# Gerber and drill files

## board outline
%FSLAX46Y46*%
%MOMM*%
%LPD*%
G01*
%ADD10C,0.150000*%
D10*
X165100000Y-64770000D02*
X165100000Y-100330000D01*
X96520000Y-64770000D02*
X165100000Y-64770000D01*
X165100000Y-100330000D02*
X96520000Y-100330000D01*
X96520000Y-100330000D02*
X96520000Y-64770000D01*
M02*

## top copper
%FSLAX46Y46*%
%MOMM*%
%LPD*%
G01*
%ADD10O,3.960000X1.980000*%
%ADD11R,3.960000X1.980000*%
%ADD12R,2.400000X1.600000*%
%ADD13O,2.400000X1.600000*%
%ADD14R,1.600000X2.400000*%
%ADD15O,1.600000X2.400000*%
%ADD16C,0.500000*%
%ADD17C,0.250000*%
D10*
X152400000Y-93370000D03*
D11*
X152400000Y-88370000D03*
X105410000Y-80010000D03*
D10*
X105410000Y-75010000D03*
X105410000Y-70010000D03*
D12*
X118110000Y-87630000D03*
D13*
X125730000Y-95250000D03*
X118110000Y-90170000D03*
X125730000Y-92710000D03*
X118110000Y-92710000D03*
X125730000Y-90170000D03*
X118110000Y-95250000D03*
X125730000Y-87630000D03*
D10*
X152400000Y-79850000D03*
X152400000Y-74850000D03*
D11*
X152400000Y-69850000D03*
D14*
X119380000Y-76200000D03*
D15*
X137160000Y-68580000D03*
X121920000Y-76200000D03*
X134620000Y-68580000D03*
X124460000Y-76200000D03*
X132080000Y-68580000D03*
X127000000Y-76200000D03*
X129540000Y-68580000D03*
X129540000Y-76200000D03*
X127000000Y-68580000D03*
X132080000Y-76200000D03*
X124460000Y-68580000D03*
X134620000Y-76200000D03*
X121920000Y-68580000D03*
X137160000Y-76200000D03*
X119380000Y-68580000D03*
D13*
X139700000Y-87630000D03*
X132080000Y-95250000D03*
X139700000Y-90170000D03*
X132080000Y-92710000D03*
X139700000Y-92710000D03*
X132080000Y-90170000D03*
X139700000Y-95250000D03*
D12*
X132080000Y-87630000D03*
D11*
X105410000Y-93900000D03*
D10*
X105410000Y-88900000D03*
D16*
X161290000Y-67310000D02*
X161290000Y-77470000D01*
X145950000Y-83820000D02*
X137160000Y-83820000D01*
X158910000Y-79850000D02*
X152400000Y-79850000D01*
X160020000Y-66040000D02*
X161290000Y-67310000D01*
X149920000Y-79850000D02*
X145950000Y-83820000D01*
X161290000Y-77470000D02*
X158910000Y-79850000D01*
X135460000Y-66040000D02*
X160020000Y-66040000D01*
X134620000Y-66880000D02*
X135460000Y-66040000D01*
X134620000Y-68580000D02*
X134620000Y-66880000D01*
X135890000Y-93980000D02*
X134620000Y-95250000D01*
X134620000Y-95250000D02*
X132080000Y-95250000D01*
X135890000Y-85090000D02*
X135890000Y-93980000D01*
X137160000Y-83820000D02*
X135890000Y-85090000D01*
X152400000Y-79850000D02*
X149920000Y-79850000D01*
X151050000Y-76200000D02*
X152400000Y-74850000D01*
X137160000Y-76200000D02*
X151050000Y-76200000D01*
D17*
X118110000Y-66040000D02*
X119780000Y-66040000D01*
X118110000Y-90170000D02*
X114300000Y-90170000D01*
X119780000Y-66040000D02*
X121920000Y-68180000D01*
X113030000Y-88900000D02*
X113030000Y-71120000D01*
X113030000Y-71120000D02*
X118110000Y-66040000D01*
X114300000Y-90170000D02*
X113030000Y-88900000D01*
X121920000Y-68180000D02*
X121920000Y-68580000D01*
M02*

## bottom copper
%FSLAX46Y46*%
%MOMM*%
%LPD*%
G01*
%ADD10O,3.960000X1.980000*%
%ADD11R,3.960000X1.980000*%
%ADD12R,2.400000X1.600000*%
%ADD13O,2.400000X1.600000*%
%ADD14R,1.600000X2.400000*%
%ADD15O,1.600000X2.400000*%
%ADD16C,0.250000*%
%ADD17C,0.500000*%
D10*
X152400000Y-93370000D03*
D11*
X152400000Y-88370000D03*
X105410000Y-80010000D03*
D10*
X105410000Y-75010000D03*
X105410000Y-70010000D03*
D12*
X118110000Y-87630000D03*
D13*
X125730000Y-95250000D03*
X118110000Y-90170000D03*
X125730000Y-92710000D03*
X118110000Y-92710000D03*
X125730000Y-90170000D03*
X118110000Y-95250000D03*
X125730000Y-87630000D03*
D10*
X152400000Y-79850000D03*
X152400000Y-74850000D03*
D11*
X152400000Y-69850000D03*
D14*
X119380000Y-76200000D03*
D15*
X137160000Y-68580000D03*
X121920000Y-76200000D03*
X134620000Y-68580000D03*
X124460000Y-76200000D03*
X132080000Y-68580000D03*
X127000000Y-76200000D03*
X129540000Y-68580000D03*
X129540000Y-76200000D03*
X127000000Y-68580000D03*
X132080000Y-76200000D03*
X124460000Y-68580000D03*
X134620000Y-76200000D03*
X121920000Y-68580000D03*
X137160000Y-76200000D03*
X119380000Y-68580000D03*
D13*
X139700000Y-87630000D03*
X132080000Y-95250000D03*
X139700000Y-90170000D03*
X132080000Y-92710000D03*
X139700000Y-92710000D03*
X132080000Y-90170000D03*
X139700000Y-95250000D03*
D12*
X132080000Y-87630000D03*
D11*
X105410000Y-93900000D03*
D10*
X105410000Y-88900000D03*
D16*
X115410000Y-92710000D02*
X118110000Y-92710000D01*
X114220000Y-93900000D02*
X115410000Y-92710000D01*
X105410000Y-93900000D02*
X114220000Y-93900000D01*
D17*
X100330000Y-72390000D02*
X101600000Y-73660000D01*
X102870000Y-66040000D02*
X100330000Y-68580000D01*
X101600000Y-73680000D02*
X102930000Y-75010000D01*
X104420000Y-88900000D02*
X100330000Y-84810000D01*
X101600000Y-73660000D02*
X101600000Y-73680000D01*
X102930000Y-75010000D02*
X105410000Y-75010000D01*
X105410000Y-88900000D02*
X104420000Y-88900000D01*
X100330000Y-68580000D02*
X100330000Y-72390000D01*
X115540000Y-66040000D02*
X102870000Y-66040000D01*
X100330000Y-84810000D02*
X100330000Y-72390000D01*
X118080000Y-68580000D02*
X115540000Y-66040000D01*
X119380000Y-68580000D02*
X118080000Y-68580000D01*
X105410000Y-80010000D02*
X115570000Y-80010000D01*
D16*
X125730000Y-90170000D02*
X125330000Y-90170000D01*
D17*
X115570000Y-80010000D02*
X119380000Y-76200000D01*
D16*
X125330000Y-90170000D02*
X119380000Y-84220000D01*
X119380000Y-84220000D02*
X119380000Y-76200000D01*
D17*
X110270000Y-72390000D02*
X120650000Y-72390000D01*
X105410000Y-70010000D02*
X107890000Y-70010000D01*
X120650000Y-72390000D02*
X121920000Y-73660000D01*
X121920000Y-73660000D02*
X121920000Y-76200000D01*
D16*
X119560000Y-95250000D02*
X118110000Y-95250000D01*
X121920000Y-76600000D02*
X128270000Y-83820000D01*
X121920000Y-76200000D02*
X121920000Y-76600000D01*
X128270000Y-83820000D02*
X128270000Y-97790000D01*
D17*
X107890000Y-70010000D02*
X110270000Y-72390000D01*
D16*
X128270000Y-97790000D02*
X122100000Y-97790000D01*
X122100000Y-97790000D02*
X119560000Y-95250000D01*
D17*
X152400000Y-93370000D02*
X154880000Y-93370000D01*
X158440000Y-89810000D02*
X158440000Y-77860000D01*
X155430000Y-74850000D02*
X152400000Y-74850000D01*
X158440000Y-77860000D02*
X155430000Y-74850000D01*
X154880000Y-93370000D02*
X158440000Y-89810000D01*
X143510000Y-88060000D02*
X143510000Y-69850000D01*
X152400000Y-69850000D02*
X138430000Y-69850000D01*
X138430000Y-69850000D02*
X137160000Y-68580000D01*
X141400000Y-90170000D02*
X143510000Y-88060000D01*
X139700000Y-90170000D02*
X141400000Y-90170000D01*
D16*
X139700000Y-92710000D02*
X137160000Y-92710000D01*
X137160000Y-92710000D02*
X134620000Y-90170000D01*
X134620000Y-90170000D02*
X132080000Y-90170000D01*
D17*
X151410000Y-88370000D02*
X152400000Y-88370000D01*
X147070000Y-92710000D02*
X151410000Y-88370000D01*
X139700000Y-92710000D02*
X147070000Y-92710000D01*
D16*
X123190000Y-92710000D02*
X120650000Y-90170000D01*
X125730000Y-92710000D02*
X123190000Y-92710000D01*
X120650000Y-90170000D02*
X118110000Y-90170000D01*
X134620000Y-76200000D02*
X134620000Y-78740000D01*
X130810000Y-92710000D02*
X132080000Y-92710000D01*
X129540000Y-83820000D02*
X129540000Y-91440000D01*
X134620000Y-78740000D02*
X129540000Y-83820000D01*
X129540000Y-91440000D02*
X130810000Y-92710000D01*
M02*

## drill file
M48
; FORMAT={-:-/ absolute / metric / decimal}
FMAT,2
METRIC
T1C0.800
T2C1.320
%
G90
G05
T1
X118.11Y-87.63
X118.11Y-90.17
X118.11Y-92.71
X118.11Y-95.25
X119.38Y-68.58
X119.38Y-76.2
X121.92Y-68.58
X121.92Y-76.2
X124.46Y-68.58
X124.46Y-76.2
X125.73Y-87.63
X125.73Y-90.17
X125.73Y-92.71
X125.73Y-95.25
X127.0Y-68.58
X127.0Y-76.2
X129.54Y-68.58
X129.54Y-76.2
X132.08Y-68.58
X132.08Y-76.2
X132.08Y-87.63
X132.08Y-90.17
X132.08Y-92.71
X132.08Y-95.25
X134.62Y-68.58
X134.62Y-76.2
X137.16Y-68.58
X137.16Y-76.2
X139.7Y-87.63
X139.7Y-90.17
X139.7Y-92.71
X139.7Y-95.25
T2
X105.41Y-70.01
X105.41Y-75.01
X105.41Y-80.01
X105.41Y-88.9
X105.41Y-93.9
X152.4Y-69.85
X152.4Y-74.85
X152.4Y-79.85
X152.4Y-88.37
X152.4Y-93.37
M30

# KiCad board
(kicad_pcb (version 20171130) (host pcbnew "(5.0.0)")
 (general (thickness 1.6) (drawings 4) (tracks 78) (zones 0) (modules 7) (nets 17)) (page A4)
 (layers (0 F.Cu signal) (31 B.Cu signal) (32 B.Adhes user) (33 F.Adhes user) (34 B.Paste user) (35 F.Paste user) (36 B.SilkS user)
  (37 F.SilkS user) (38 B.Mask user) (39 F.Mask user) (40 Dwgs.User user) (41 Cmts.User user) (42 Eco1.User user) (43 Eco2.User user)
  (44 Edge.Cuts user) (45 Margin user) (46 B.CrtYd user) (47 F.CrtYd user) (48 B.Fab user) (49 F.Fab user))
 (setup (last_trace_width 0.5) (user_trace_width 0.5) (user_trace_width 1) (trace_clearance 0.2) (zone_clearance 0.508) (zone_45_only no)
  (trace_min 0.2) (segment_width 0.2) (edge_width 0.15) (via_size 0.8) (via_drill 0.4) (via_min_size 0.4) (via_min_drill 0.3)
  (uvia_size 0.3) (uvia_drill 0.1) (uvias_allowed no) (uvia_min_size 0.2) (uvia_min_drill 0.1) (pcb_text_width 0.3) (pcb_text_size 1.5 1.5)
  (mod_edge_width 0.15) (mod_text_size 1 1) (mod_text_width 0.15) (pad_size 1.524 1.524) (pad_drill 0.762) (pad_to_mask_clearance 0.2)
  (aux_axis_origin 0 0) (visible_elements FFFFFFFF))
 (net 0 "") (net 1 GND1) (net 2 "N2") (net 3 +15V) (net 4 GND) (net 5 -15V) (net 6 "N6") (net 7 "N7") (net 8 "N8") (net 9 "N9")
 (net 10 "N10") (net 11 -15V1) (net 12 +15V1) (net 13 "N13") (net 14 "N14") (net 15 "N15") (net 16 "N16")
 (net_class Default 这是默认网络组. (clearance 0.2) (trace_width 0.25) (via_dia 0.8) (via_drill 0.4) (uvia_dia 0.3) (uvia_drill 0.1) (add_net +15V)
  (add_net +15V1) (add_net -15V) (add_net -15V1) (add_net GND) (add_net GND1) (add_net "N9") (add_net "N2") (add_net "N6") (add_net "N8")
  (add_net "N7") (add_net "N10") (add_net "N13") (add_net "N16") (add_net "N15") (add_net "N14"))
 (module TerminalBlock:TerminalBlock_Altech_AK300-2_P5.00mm (layer F.Cu) (at 152.4 88.37 270)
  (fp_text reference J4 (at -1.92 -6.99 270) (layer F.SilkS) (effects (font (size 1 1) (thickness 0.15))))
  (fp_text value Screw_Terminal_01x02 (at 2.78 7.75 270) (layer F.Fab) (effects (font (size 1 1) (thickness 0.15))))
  (pad 2 thru_hole oval (at 5 0 270) (size 1.98 3.96) (drill 1.32) (layers *.Cu *.Mask) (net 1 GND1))
  (pad 1 thru_hole rect (at 0 0 270) (size 1.98 3.96) (drill 1.32) (layers *.Cu *.Mask) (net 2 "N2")))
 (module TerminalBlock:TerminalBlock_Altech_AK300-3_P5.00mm (layer F.Cu) (at 105.41 80.01 90)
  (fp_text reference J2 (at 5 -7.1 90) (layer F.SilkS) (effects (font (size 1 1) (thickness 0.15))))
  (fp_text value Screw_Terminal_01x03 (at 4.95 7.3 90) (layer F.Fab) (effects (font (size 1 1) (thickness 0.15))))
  (pad 1 thru_hole rect (at 0 0 90) (size 1.98 3.96) (drill 1.32) (layers *.Cu *.Mask) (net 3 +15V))
  (pad 2 thru_hole oval (at 5 0 90) (size 1.98 3.96) (drill 1.32) (layers *.Cu *.Mask) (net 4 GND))
  (pad 3 thru_hole oval (at 10 0 90) (size 1.98 3.96) (drill 1.32) (layers *.Cu *.Mask) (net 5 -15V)))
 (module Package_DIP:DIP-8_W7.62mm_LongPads (layer F.Cu) (at 118.11 87.63)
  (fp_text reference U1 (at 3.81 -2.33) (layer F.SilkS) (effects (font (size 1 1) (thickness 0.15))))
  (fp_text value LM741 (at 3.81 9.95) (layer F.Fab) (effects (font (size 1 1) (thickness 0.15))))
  (pad 1 thru_hole rect (at 0 0) (size 2.4 1.6) (drill 0.8) (layers *.Cu *.Mask) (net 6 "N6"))
  (pad 5 thru_hole oval (at 7.62 7.62) (size 2.4 1.6) (drill 0.8) (layers *.Cu *.Mask) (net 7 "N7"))
  (pad 2 thru_hole oval (at 0 2.54) (size 2.4 1.6) (drill 0.8) (layers *.Cu *.Mask) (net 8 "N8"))
  (pad 6 thru_hole oval (at 7.62 5.08) (size 2.4 1.6) (drill 0.8) (layers *.Cu *.Mask) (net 8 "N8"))
  (pad 3 thru_hole oval (at 0 5.08) (size 2.4 1.6) (drill 0.8) (layers *.Cu *.Mask) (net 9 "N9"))
  (pad 7 thru_hole oval (at 7.62 2.54) (size 2.4 1.6) (drill 0.8) (layers *.Cu *.Mask) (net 3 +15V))
  (pad 4 thru_hole oval (at 0 7.62) (size 2.4 1.6) (drill 0.8) (layers *.Cu *.Mask) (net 5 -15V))
  (pad 8 thru_hole oval (at 7.62 0) (size 2.4 1.6) (drill 0.8) (layers *.Cu *.Mask) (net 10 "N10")))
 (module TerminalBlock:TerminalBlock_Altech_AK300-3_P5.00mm (layer F.Cu) (at 152.4 69.85 270)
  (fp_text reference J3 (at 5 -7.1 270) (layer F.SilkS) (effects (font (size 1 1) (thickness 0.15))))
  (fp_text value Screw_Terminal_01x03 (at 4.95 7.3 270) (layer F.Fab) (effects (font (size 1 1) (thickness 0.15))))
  (pad 3 thru_hole oval (at 10 0 270) (size 1.98 3.96) (drill 1.32) (layers *.Cu *.Mask) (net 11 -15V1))
  (pad 2 thru_hole oval (at 5 0 270) (size 1.98 3.96) (drill 1.32) (layers *.Cu *.Mask) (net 1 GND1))
  (pad 1 thru_hole rect (at 0 0 270) (size 1.98 3.96) (drill 1.32) (layers *.Cu *.Mask) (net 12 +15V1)))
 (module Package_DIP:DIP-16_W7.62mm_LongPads (layer F.Cu) (at 119.38 76.2 90)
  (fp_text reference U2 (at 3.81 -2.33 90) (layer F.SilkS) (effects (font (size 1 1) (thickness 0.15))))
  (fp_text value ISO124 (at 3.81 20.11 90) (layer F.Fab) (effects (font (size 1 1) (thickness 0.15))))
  (pad 1 thru_hole rect (at 0 0 90) (size 2.4 1.6) (drill 0.8) (layers *.Cu *.Mask) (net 3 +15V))
  (pad 9 thru_hole oval (at 7.62 17.78 90) (size 2.4 1.6) (drill 0.8) (layers *.Cu *.Mask) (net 12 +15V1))
  (pad 2 thru_hole oval (at 0 2.54 90) (size 2.4 1.6) (drill 0.8) (layers *.Cu *.Mask) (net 5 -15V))
  (pad 10 thru_hole oval (at 7.62 15.24 90) (size 2.4 1.6) (drill 0.8) (layers *.Cu *.Mask) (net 11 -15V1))
  (pad 3 thru_hole oval (at 0 5.08 90) (size 2.4 1.6) (drill 0.8) (layers *.Cu *.Mask))
  (pad 11 thru_hole oval (at 7.62 12.7 90) (size 2.4 1.6) (drill 0.8) (layers *.Cu *.Mask))
  (pad 4 thru_hole oval (at 0 7.62 90) (size 2.4 1.6) (drill 0.8) (layers *.Cu *.Mask))
  (pad 12 thru_hole oval (at 7.62 10.16 90) (size 2.4 1.6) (drill 0.8) (layers *.Cu *.Mask))
  (pad 5 thru_hole oval (at 0 10.16 90) (size 2.4 1.6) (drill 0.8) (layers *.Cu *.Mask))
  (pad 13 thru_hole oval (at 7.62 7.62 90) (size 2.4 1.6) (drill 0.8) (layers *.Cu *.Mask))
  (pad 6 thru_hole oval (at 0 12.7 90) (size 2.4 1.6) (drill 0.8) (layers *.Cu *.Mask))
  (pad 14 thru_hole oval (at 7.62 5.08 90) (size 2.4 1.6) (drill 0.8) (layers *.Cu *.Mask))
  (pad 7 thru_hole oval (at 0 15.24 90) (size 2.4 1.6) (drill 0.8) (layers *.Cu *.Mask) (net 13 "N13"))
  (pad 15 thru_hole oval (at 7.62 2.54 90) (size 2.4 1.6) (drill 0.8) (layers *.Cu *.Mask) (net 8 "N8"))
  (pad 8 thru_hole oval (at 0 17.78 90) (size 2.4 1.6) (drill 0.8) (layers *.Cu *.Mask) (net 1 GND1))
  (pad 16 thru_hole oval (at 7.62 0 90) (size 2.4 1.6) (drill 0.8) (layers *.Cu *.Mask) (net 4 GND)))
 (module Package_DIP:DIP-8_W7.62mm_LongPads (layer F.Cu) (at 132.08 87.63)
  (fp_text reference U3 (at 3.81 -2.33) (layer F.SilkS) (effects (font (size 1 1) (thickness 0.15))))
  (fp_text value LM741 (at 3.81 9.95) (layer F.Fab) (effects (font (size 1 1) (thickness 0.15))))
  (pad 8 thru_hole oval (at 7.62 0) (size 2.4 1.6) (drill 0.8) (layers *.Cu *.Mask) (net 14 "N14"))
  (pad 4 thru_hole oval (at 0 7.62) (size 2.4 1.6) (drill 0.8) (layers *.Cu *.Mask) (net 11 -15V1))
  (pad 7 thru_hole oval (at 7.62 2.54) (size 2.4 1.6) (drill 0.8) (layers *.Cu *.Mask) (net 12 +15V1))
  (pad 3 thru_hole oval (at 0 5.08) (size 2.4 1.6) (drill 0.8) (layers *.Cu *.Mask) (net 13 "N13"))
  (pad 6 thru_hole oval (at 7.62 5.08) (size 2.4 1.6) (drill 0.8) (layers *.Cu *.Mask) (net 2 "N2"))
  (pad 2 thru_hole oval (at 0 2.54) (size 2.4 1.6) (drill 0.8) (layers *.Cu *.Mask) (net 2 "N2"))
  (pad 5 thru_hole oval (at 7.62 7.62) (size 2.4 1.6) (drill 0.8) (layers *.Cu *.Mask) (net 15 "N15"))
  (pad 1 thru_hole rect (at 0 0) (size 2.4 1.6) (drill 0.8) (layers *.Cu *.Mask) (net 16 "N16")))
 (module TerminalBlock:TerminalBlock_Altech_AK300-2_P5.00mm (layer F.Cu) (at 105.41 93.9 90)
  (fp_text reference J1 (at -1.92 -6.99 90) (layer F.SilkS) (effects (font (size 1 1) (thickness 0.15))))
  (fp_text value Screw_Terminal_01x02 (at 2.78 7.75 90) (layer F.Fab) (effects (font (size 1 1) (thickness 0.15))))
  (pad 1 thru_hole rect (at 0 0 90) (size 1.98 3.96) (drill 1.32) (layers *.Cu *.Mask) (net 9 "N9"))
  (pad 2 thru_hole oval (at 5 0 90) (size 1.98 3.96) (drill 1.32) (layers *.Cu *.Mask) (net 4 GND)))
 (gr_line (start 165.1 64.77) (end 165.1 100.33) (layer Edge.Cuts) (width 0.15))
 (gr_line (start 96.52 64.77) (end 165.1 64.77) (layer Edge.Cuts) (width 0.15))
 (gr_line (start 165.1 100.33) (end 96.52 100.33) (layer Edge.Cuts) (width 0.15))
 (gr_line (start 96.52 100.33) (end 96.52 64.77) (layer Edge.Cuts) (width 0.15))
 (segment (start 115.41 92.71) (end 118.11 92.71) (width 0.25) (layer B.Cu) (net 9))
 (segment (start 114.22 93.9) (end 115.41 92.71) (width 0.25) (layer B.Cu) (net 9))
 (segment (start 105.41 93.9) (end 114.22 93.9) (width 0.25) (layer B.Cu) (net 9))
 (segment (start 100.33 72.39) (end 101.6 73.66) (width 0.5) (layer B.Cu) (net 4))
 (segment (start 102.87 66.04) (end 100.33 68.58) (width 0.5) (layer B.Cu) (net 4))
 (segment (start 101.6 73.68) (end 102.93 75.01) (width 0.5) (layer B.Cu) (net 4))
 (segment (start 104.42 88.9) (end 100.33 84.81) (width 0.5) (layer B.Cu) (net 4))
 (segment (start 101.6 73.66) (end 101.6 73.68) (width 0.5) (layer B.Cu) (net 4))
 (segment (start 102.93 75.01) (end 105.41 75.01) (width 0.5) (layer B.Cu) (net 4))
 (segment (start 105.41 88.9) (end 104.42 88.9) (width 0.5) (layer B.Cu) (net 4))
 (segment (start 100.33 68.58) (end 100.33 72.39) (width 0.5) (layer B.Cu) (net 4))
 (segment (start 115.54 66.04) (end 102.87 66.04) (width 0.5) (layer B.Cu) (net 4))
 (segment (start 100.33 84.81) (end 100.33 72.39) (width 0.5) (layer B.Cu) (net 4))
 (segment (start 118.08 68.58) (end 115.54 66.04) (width 0.5) (layer B.Cu) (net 4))
 (segment (start 119.38 68.58) (end 118.08 68.58) (width 0.5) (layer B.Cu) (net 4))
 (segment (start 105.41 80.01) (end 115.57 80.01) (width 0.5) (layer B.Cu) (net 3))
 (segment (start 125.73 90.17) (end 125.33 90.17) (width 0.25) (layer B.Cu) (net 3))
 (segment (start 115.57 80.01) (end 119.38 76.2) (width 0.5) (layer B.Cu) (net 3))
 (segment (start 125.33 90.17) (end 119.38 84.22) (width 0.25) (layer B.Cu) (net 3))
 (segment (start 119.38 84.22) (end 119.38 76.2) (width 0.25) (layer B.Cu) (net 3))
 (segment (start 110.27 72.39) (end 120.65 72.39) (width 0.5) (layer B.Cu) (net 5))
 (segment (start 105.41 70.01) (end 107.89 70.01) (width 0.5) (layer B.Cu) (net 5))
 (segment (start 120.65 72.39) (end 121.92 73.66) (width 0.5) (layer B.Cu) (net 5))
 (segment (start 121.92 73.66) (end 121.92 76.2) (width 0.5) (layer B.Cu) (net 5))
 (segment (start 119.56 95.25) (end 118.11 95.25) (width 0.25) (layer B.Cu) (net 5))
 (segment (start 121.92 76.6) (end 128.27 83.82) (width 0.25) (layer B.Cu) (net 5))
 (segment (start 121.92 76.2) (end 121.92 76.6) (width 0.25) (layer B.Cu) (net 5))
 (segment (start 128.27 83.82) (end 128.27 97.79) (width 0.25) (layer B.Cu) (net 5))
 (segment (start 107.89 70.01) (end 110.27 72.39) (width 0.5) (layer B.Cu) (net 5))
 (segment (start 128.27 97.79) (end 122.1 97.79) (width 0.25) (layer B.Cu) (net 5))
 (segment (start 122.1 97.79) (end 119.56 95.25) (width 0.25) (layer B.Cu) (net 5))
 (segment (start 161.29 67.31) (end 161.29 77.47) (width 0.5) (layer F.Cu) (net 11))
 (segment (start 145.95 83.82) (end 137.16 83.82) (width 0.5) (layer F.Cu) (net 11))
 (segment (start 158.91 79.85) (end 152.4 79.85) (width 0.5) (layer F.Cu) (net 11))
 (segment (start 160.02 66.04) (end 161.29 67.31) (width 0.5) (layer F.Cu) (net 11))
 (segment (start 149.92 79.85) (end 145.95 83.82) (width 0.5) (layer F.Cu) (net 11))
 (segment (start 161.29 77.47) (end 158.91 79.85) (width 0.5) (layer F.Cu) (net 11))
 (segment (start 135.46 66.04) (end 160.02 66.04) (width 0.5) (layer F.Cu) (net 11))
 (segment (start 134.62 66.88) (end 135.46 66.04) (width 0.5) (layer F.Cu) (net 11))
 (segment (start 134.62 68.58) (end 134.62 66.88) (width 0.5) (layer F.Cu) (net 11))
 (segment (start 135.89 93.98) (end 134.62 95.25) (width 0.5) (layer F.Cu) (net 11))
 (segment (start 134.62 95.25) (end 132.08 95.25) (width 0.5) (layer F.Cu) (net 11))
 (segment (start 135.89 85.09) (end 135.89 93.98) (width 0.5) (layer F.Cu) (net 11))
 (segment (start 137.16 83.82) (end 135.89 85.09) (width 0.5) (layer F.Cu) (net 11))
 (segment (start 152.4 79.85) (end 149.92 79.85) (width 0.5) (layer F.Cu) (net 11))
 (segment (start 151.05 76.2) (end 152.4 74.85) (width 0.5) (layer F.Cu) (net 1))
 (segment (start 137.16 76.2) (end 151.05 76.2) (width 0.5) (layer F.Cu) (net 1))
 (segment (start 152.4 93.37) (end 154.88 93.37) (width 0.5) (layer B.Cu) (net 1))
 (segment (start 158.44 89.81) (end 158.44 77.86) (width 0.5) (layer B.Cu) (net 1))
 (segment (start 155.43 74.85) (end 152.4 74.85) (width 0.5) (layer B.Cu) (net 1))
 (segment (start 158.44 77.86) (end 155.43 74.85) (width 0.5) (layer B.Cu) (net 1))
 (segment (start 154.88 93.37) (end 158.44 89.81) (width 0.5) (layer B.Cu) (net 1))
 (segment (start 143.51 88.06) (end 143.51 69.85) (width 0.5) (layer B.Cu) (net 12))
 (segment (start 152.4 69.85) (end 138.43 69.85) (width 0.5) (layer B.Cu) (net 12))
 (segment (start 138.43 69.85) (end 137.16 68.58) (width 0.5) (layer B.Cu) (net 12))
 (segment (start 141.4 90.17) (end 143.51 88.06) (width 0.5) (layer B.Cu) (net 12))
 (segment (start 139.7 90.17) (end 141.4 90.17) (width 0.5) (layer B.Cu) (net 12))
 (segment (start 139.7 92.71) (end 137.16 92.71) (width 0.25) (layer B.Cu) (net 2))
 (segment (start 137.16 92.71) (end 134.62 90.17) (width 0.25) (layer B.Cu) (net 2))
 (segment (start 134.62 90.17) (end 132.08 90.17) (width 0.25) (layer B.Cu) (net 2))
 (segment (start 151.41 88.37) (end 152.4 88.37) (width 0.5) (layer B.Cu) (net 2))
 (segment (start 147.07 92.71) (end 151.41 88.37) (width 0.5) (layer B.Cu) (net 2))
 (segment (start 139.7 92.71) (end 147.07 92.71) (width 0.5) (layer B.Cu) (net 2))
 (segment (start 123.19 92.71) (end 120.65 90.17) (width 0.25) (layer B.Cu) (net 8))
 (segment (start 118.11 66.04) (end 119.78 66.04) (width 0.25) (layer F.Cu) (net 8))
 (segment (start 118.11 90.17) (end 114.3 90.17) (width 0.25) (layer F.Cu) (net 8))
 (segment (start 119.78 66.04) (end 121.92 68.18) (width 0.25) (layer F.Cu) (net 8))
 (segment (start 125.73 92.71) (end 123.19 92.71) (width 0.25) (layer B.Cu) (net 8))
 (segment (start 113.03 88.9) (end 113.03 71.12) (width 0.25) (layer F.Cu) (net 8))
 (segment (start 113.03 71.12) (end 118.11 66.04) (width 0.25) (layer F.Cu) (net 8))
 (segment (start 114.3 90.17) (end 113.03 88.9) (width 0.25) (layer F.Cu) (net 8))
 (segment (start 121.92 68.18) (end 121.92 68.58) (width 0.25) (layer F.Cu) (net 8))
 (segment (start 120.65 90.17) (end 118.11 90.17) (width 0.25) (layer B.Cu) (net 8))
 (segment (start 134.62 76.2) (end 134.62 78.74) (width 0.25) (layer B.Cu) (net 13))
 (segment (start 130.81 92.71) (end 132.08 92.71) (width 0.25) (layer B.Cu) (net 13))
 (segment (start 129.54 83.82) (end 129.54 91.44) (width 0.25) (layer B.Cu) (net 13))
 (segment (start 134.62 78.74) (end 129.54 83.82) (width 0.25) (layer B.Cu) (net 13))
 (segment (start 129.54 91.44) (end 130.81 92.71) (width 0.25) (layer B.Cu) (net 13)))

